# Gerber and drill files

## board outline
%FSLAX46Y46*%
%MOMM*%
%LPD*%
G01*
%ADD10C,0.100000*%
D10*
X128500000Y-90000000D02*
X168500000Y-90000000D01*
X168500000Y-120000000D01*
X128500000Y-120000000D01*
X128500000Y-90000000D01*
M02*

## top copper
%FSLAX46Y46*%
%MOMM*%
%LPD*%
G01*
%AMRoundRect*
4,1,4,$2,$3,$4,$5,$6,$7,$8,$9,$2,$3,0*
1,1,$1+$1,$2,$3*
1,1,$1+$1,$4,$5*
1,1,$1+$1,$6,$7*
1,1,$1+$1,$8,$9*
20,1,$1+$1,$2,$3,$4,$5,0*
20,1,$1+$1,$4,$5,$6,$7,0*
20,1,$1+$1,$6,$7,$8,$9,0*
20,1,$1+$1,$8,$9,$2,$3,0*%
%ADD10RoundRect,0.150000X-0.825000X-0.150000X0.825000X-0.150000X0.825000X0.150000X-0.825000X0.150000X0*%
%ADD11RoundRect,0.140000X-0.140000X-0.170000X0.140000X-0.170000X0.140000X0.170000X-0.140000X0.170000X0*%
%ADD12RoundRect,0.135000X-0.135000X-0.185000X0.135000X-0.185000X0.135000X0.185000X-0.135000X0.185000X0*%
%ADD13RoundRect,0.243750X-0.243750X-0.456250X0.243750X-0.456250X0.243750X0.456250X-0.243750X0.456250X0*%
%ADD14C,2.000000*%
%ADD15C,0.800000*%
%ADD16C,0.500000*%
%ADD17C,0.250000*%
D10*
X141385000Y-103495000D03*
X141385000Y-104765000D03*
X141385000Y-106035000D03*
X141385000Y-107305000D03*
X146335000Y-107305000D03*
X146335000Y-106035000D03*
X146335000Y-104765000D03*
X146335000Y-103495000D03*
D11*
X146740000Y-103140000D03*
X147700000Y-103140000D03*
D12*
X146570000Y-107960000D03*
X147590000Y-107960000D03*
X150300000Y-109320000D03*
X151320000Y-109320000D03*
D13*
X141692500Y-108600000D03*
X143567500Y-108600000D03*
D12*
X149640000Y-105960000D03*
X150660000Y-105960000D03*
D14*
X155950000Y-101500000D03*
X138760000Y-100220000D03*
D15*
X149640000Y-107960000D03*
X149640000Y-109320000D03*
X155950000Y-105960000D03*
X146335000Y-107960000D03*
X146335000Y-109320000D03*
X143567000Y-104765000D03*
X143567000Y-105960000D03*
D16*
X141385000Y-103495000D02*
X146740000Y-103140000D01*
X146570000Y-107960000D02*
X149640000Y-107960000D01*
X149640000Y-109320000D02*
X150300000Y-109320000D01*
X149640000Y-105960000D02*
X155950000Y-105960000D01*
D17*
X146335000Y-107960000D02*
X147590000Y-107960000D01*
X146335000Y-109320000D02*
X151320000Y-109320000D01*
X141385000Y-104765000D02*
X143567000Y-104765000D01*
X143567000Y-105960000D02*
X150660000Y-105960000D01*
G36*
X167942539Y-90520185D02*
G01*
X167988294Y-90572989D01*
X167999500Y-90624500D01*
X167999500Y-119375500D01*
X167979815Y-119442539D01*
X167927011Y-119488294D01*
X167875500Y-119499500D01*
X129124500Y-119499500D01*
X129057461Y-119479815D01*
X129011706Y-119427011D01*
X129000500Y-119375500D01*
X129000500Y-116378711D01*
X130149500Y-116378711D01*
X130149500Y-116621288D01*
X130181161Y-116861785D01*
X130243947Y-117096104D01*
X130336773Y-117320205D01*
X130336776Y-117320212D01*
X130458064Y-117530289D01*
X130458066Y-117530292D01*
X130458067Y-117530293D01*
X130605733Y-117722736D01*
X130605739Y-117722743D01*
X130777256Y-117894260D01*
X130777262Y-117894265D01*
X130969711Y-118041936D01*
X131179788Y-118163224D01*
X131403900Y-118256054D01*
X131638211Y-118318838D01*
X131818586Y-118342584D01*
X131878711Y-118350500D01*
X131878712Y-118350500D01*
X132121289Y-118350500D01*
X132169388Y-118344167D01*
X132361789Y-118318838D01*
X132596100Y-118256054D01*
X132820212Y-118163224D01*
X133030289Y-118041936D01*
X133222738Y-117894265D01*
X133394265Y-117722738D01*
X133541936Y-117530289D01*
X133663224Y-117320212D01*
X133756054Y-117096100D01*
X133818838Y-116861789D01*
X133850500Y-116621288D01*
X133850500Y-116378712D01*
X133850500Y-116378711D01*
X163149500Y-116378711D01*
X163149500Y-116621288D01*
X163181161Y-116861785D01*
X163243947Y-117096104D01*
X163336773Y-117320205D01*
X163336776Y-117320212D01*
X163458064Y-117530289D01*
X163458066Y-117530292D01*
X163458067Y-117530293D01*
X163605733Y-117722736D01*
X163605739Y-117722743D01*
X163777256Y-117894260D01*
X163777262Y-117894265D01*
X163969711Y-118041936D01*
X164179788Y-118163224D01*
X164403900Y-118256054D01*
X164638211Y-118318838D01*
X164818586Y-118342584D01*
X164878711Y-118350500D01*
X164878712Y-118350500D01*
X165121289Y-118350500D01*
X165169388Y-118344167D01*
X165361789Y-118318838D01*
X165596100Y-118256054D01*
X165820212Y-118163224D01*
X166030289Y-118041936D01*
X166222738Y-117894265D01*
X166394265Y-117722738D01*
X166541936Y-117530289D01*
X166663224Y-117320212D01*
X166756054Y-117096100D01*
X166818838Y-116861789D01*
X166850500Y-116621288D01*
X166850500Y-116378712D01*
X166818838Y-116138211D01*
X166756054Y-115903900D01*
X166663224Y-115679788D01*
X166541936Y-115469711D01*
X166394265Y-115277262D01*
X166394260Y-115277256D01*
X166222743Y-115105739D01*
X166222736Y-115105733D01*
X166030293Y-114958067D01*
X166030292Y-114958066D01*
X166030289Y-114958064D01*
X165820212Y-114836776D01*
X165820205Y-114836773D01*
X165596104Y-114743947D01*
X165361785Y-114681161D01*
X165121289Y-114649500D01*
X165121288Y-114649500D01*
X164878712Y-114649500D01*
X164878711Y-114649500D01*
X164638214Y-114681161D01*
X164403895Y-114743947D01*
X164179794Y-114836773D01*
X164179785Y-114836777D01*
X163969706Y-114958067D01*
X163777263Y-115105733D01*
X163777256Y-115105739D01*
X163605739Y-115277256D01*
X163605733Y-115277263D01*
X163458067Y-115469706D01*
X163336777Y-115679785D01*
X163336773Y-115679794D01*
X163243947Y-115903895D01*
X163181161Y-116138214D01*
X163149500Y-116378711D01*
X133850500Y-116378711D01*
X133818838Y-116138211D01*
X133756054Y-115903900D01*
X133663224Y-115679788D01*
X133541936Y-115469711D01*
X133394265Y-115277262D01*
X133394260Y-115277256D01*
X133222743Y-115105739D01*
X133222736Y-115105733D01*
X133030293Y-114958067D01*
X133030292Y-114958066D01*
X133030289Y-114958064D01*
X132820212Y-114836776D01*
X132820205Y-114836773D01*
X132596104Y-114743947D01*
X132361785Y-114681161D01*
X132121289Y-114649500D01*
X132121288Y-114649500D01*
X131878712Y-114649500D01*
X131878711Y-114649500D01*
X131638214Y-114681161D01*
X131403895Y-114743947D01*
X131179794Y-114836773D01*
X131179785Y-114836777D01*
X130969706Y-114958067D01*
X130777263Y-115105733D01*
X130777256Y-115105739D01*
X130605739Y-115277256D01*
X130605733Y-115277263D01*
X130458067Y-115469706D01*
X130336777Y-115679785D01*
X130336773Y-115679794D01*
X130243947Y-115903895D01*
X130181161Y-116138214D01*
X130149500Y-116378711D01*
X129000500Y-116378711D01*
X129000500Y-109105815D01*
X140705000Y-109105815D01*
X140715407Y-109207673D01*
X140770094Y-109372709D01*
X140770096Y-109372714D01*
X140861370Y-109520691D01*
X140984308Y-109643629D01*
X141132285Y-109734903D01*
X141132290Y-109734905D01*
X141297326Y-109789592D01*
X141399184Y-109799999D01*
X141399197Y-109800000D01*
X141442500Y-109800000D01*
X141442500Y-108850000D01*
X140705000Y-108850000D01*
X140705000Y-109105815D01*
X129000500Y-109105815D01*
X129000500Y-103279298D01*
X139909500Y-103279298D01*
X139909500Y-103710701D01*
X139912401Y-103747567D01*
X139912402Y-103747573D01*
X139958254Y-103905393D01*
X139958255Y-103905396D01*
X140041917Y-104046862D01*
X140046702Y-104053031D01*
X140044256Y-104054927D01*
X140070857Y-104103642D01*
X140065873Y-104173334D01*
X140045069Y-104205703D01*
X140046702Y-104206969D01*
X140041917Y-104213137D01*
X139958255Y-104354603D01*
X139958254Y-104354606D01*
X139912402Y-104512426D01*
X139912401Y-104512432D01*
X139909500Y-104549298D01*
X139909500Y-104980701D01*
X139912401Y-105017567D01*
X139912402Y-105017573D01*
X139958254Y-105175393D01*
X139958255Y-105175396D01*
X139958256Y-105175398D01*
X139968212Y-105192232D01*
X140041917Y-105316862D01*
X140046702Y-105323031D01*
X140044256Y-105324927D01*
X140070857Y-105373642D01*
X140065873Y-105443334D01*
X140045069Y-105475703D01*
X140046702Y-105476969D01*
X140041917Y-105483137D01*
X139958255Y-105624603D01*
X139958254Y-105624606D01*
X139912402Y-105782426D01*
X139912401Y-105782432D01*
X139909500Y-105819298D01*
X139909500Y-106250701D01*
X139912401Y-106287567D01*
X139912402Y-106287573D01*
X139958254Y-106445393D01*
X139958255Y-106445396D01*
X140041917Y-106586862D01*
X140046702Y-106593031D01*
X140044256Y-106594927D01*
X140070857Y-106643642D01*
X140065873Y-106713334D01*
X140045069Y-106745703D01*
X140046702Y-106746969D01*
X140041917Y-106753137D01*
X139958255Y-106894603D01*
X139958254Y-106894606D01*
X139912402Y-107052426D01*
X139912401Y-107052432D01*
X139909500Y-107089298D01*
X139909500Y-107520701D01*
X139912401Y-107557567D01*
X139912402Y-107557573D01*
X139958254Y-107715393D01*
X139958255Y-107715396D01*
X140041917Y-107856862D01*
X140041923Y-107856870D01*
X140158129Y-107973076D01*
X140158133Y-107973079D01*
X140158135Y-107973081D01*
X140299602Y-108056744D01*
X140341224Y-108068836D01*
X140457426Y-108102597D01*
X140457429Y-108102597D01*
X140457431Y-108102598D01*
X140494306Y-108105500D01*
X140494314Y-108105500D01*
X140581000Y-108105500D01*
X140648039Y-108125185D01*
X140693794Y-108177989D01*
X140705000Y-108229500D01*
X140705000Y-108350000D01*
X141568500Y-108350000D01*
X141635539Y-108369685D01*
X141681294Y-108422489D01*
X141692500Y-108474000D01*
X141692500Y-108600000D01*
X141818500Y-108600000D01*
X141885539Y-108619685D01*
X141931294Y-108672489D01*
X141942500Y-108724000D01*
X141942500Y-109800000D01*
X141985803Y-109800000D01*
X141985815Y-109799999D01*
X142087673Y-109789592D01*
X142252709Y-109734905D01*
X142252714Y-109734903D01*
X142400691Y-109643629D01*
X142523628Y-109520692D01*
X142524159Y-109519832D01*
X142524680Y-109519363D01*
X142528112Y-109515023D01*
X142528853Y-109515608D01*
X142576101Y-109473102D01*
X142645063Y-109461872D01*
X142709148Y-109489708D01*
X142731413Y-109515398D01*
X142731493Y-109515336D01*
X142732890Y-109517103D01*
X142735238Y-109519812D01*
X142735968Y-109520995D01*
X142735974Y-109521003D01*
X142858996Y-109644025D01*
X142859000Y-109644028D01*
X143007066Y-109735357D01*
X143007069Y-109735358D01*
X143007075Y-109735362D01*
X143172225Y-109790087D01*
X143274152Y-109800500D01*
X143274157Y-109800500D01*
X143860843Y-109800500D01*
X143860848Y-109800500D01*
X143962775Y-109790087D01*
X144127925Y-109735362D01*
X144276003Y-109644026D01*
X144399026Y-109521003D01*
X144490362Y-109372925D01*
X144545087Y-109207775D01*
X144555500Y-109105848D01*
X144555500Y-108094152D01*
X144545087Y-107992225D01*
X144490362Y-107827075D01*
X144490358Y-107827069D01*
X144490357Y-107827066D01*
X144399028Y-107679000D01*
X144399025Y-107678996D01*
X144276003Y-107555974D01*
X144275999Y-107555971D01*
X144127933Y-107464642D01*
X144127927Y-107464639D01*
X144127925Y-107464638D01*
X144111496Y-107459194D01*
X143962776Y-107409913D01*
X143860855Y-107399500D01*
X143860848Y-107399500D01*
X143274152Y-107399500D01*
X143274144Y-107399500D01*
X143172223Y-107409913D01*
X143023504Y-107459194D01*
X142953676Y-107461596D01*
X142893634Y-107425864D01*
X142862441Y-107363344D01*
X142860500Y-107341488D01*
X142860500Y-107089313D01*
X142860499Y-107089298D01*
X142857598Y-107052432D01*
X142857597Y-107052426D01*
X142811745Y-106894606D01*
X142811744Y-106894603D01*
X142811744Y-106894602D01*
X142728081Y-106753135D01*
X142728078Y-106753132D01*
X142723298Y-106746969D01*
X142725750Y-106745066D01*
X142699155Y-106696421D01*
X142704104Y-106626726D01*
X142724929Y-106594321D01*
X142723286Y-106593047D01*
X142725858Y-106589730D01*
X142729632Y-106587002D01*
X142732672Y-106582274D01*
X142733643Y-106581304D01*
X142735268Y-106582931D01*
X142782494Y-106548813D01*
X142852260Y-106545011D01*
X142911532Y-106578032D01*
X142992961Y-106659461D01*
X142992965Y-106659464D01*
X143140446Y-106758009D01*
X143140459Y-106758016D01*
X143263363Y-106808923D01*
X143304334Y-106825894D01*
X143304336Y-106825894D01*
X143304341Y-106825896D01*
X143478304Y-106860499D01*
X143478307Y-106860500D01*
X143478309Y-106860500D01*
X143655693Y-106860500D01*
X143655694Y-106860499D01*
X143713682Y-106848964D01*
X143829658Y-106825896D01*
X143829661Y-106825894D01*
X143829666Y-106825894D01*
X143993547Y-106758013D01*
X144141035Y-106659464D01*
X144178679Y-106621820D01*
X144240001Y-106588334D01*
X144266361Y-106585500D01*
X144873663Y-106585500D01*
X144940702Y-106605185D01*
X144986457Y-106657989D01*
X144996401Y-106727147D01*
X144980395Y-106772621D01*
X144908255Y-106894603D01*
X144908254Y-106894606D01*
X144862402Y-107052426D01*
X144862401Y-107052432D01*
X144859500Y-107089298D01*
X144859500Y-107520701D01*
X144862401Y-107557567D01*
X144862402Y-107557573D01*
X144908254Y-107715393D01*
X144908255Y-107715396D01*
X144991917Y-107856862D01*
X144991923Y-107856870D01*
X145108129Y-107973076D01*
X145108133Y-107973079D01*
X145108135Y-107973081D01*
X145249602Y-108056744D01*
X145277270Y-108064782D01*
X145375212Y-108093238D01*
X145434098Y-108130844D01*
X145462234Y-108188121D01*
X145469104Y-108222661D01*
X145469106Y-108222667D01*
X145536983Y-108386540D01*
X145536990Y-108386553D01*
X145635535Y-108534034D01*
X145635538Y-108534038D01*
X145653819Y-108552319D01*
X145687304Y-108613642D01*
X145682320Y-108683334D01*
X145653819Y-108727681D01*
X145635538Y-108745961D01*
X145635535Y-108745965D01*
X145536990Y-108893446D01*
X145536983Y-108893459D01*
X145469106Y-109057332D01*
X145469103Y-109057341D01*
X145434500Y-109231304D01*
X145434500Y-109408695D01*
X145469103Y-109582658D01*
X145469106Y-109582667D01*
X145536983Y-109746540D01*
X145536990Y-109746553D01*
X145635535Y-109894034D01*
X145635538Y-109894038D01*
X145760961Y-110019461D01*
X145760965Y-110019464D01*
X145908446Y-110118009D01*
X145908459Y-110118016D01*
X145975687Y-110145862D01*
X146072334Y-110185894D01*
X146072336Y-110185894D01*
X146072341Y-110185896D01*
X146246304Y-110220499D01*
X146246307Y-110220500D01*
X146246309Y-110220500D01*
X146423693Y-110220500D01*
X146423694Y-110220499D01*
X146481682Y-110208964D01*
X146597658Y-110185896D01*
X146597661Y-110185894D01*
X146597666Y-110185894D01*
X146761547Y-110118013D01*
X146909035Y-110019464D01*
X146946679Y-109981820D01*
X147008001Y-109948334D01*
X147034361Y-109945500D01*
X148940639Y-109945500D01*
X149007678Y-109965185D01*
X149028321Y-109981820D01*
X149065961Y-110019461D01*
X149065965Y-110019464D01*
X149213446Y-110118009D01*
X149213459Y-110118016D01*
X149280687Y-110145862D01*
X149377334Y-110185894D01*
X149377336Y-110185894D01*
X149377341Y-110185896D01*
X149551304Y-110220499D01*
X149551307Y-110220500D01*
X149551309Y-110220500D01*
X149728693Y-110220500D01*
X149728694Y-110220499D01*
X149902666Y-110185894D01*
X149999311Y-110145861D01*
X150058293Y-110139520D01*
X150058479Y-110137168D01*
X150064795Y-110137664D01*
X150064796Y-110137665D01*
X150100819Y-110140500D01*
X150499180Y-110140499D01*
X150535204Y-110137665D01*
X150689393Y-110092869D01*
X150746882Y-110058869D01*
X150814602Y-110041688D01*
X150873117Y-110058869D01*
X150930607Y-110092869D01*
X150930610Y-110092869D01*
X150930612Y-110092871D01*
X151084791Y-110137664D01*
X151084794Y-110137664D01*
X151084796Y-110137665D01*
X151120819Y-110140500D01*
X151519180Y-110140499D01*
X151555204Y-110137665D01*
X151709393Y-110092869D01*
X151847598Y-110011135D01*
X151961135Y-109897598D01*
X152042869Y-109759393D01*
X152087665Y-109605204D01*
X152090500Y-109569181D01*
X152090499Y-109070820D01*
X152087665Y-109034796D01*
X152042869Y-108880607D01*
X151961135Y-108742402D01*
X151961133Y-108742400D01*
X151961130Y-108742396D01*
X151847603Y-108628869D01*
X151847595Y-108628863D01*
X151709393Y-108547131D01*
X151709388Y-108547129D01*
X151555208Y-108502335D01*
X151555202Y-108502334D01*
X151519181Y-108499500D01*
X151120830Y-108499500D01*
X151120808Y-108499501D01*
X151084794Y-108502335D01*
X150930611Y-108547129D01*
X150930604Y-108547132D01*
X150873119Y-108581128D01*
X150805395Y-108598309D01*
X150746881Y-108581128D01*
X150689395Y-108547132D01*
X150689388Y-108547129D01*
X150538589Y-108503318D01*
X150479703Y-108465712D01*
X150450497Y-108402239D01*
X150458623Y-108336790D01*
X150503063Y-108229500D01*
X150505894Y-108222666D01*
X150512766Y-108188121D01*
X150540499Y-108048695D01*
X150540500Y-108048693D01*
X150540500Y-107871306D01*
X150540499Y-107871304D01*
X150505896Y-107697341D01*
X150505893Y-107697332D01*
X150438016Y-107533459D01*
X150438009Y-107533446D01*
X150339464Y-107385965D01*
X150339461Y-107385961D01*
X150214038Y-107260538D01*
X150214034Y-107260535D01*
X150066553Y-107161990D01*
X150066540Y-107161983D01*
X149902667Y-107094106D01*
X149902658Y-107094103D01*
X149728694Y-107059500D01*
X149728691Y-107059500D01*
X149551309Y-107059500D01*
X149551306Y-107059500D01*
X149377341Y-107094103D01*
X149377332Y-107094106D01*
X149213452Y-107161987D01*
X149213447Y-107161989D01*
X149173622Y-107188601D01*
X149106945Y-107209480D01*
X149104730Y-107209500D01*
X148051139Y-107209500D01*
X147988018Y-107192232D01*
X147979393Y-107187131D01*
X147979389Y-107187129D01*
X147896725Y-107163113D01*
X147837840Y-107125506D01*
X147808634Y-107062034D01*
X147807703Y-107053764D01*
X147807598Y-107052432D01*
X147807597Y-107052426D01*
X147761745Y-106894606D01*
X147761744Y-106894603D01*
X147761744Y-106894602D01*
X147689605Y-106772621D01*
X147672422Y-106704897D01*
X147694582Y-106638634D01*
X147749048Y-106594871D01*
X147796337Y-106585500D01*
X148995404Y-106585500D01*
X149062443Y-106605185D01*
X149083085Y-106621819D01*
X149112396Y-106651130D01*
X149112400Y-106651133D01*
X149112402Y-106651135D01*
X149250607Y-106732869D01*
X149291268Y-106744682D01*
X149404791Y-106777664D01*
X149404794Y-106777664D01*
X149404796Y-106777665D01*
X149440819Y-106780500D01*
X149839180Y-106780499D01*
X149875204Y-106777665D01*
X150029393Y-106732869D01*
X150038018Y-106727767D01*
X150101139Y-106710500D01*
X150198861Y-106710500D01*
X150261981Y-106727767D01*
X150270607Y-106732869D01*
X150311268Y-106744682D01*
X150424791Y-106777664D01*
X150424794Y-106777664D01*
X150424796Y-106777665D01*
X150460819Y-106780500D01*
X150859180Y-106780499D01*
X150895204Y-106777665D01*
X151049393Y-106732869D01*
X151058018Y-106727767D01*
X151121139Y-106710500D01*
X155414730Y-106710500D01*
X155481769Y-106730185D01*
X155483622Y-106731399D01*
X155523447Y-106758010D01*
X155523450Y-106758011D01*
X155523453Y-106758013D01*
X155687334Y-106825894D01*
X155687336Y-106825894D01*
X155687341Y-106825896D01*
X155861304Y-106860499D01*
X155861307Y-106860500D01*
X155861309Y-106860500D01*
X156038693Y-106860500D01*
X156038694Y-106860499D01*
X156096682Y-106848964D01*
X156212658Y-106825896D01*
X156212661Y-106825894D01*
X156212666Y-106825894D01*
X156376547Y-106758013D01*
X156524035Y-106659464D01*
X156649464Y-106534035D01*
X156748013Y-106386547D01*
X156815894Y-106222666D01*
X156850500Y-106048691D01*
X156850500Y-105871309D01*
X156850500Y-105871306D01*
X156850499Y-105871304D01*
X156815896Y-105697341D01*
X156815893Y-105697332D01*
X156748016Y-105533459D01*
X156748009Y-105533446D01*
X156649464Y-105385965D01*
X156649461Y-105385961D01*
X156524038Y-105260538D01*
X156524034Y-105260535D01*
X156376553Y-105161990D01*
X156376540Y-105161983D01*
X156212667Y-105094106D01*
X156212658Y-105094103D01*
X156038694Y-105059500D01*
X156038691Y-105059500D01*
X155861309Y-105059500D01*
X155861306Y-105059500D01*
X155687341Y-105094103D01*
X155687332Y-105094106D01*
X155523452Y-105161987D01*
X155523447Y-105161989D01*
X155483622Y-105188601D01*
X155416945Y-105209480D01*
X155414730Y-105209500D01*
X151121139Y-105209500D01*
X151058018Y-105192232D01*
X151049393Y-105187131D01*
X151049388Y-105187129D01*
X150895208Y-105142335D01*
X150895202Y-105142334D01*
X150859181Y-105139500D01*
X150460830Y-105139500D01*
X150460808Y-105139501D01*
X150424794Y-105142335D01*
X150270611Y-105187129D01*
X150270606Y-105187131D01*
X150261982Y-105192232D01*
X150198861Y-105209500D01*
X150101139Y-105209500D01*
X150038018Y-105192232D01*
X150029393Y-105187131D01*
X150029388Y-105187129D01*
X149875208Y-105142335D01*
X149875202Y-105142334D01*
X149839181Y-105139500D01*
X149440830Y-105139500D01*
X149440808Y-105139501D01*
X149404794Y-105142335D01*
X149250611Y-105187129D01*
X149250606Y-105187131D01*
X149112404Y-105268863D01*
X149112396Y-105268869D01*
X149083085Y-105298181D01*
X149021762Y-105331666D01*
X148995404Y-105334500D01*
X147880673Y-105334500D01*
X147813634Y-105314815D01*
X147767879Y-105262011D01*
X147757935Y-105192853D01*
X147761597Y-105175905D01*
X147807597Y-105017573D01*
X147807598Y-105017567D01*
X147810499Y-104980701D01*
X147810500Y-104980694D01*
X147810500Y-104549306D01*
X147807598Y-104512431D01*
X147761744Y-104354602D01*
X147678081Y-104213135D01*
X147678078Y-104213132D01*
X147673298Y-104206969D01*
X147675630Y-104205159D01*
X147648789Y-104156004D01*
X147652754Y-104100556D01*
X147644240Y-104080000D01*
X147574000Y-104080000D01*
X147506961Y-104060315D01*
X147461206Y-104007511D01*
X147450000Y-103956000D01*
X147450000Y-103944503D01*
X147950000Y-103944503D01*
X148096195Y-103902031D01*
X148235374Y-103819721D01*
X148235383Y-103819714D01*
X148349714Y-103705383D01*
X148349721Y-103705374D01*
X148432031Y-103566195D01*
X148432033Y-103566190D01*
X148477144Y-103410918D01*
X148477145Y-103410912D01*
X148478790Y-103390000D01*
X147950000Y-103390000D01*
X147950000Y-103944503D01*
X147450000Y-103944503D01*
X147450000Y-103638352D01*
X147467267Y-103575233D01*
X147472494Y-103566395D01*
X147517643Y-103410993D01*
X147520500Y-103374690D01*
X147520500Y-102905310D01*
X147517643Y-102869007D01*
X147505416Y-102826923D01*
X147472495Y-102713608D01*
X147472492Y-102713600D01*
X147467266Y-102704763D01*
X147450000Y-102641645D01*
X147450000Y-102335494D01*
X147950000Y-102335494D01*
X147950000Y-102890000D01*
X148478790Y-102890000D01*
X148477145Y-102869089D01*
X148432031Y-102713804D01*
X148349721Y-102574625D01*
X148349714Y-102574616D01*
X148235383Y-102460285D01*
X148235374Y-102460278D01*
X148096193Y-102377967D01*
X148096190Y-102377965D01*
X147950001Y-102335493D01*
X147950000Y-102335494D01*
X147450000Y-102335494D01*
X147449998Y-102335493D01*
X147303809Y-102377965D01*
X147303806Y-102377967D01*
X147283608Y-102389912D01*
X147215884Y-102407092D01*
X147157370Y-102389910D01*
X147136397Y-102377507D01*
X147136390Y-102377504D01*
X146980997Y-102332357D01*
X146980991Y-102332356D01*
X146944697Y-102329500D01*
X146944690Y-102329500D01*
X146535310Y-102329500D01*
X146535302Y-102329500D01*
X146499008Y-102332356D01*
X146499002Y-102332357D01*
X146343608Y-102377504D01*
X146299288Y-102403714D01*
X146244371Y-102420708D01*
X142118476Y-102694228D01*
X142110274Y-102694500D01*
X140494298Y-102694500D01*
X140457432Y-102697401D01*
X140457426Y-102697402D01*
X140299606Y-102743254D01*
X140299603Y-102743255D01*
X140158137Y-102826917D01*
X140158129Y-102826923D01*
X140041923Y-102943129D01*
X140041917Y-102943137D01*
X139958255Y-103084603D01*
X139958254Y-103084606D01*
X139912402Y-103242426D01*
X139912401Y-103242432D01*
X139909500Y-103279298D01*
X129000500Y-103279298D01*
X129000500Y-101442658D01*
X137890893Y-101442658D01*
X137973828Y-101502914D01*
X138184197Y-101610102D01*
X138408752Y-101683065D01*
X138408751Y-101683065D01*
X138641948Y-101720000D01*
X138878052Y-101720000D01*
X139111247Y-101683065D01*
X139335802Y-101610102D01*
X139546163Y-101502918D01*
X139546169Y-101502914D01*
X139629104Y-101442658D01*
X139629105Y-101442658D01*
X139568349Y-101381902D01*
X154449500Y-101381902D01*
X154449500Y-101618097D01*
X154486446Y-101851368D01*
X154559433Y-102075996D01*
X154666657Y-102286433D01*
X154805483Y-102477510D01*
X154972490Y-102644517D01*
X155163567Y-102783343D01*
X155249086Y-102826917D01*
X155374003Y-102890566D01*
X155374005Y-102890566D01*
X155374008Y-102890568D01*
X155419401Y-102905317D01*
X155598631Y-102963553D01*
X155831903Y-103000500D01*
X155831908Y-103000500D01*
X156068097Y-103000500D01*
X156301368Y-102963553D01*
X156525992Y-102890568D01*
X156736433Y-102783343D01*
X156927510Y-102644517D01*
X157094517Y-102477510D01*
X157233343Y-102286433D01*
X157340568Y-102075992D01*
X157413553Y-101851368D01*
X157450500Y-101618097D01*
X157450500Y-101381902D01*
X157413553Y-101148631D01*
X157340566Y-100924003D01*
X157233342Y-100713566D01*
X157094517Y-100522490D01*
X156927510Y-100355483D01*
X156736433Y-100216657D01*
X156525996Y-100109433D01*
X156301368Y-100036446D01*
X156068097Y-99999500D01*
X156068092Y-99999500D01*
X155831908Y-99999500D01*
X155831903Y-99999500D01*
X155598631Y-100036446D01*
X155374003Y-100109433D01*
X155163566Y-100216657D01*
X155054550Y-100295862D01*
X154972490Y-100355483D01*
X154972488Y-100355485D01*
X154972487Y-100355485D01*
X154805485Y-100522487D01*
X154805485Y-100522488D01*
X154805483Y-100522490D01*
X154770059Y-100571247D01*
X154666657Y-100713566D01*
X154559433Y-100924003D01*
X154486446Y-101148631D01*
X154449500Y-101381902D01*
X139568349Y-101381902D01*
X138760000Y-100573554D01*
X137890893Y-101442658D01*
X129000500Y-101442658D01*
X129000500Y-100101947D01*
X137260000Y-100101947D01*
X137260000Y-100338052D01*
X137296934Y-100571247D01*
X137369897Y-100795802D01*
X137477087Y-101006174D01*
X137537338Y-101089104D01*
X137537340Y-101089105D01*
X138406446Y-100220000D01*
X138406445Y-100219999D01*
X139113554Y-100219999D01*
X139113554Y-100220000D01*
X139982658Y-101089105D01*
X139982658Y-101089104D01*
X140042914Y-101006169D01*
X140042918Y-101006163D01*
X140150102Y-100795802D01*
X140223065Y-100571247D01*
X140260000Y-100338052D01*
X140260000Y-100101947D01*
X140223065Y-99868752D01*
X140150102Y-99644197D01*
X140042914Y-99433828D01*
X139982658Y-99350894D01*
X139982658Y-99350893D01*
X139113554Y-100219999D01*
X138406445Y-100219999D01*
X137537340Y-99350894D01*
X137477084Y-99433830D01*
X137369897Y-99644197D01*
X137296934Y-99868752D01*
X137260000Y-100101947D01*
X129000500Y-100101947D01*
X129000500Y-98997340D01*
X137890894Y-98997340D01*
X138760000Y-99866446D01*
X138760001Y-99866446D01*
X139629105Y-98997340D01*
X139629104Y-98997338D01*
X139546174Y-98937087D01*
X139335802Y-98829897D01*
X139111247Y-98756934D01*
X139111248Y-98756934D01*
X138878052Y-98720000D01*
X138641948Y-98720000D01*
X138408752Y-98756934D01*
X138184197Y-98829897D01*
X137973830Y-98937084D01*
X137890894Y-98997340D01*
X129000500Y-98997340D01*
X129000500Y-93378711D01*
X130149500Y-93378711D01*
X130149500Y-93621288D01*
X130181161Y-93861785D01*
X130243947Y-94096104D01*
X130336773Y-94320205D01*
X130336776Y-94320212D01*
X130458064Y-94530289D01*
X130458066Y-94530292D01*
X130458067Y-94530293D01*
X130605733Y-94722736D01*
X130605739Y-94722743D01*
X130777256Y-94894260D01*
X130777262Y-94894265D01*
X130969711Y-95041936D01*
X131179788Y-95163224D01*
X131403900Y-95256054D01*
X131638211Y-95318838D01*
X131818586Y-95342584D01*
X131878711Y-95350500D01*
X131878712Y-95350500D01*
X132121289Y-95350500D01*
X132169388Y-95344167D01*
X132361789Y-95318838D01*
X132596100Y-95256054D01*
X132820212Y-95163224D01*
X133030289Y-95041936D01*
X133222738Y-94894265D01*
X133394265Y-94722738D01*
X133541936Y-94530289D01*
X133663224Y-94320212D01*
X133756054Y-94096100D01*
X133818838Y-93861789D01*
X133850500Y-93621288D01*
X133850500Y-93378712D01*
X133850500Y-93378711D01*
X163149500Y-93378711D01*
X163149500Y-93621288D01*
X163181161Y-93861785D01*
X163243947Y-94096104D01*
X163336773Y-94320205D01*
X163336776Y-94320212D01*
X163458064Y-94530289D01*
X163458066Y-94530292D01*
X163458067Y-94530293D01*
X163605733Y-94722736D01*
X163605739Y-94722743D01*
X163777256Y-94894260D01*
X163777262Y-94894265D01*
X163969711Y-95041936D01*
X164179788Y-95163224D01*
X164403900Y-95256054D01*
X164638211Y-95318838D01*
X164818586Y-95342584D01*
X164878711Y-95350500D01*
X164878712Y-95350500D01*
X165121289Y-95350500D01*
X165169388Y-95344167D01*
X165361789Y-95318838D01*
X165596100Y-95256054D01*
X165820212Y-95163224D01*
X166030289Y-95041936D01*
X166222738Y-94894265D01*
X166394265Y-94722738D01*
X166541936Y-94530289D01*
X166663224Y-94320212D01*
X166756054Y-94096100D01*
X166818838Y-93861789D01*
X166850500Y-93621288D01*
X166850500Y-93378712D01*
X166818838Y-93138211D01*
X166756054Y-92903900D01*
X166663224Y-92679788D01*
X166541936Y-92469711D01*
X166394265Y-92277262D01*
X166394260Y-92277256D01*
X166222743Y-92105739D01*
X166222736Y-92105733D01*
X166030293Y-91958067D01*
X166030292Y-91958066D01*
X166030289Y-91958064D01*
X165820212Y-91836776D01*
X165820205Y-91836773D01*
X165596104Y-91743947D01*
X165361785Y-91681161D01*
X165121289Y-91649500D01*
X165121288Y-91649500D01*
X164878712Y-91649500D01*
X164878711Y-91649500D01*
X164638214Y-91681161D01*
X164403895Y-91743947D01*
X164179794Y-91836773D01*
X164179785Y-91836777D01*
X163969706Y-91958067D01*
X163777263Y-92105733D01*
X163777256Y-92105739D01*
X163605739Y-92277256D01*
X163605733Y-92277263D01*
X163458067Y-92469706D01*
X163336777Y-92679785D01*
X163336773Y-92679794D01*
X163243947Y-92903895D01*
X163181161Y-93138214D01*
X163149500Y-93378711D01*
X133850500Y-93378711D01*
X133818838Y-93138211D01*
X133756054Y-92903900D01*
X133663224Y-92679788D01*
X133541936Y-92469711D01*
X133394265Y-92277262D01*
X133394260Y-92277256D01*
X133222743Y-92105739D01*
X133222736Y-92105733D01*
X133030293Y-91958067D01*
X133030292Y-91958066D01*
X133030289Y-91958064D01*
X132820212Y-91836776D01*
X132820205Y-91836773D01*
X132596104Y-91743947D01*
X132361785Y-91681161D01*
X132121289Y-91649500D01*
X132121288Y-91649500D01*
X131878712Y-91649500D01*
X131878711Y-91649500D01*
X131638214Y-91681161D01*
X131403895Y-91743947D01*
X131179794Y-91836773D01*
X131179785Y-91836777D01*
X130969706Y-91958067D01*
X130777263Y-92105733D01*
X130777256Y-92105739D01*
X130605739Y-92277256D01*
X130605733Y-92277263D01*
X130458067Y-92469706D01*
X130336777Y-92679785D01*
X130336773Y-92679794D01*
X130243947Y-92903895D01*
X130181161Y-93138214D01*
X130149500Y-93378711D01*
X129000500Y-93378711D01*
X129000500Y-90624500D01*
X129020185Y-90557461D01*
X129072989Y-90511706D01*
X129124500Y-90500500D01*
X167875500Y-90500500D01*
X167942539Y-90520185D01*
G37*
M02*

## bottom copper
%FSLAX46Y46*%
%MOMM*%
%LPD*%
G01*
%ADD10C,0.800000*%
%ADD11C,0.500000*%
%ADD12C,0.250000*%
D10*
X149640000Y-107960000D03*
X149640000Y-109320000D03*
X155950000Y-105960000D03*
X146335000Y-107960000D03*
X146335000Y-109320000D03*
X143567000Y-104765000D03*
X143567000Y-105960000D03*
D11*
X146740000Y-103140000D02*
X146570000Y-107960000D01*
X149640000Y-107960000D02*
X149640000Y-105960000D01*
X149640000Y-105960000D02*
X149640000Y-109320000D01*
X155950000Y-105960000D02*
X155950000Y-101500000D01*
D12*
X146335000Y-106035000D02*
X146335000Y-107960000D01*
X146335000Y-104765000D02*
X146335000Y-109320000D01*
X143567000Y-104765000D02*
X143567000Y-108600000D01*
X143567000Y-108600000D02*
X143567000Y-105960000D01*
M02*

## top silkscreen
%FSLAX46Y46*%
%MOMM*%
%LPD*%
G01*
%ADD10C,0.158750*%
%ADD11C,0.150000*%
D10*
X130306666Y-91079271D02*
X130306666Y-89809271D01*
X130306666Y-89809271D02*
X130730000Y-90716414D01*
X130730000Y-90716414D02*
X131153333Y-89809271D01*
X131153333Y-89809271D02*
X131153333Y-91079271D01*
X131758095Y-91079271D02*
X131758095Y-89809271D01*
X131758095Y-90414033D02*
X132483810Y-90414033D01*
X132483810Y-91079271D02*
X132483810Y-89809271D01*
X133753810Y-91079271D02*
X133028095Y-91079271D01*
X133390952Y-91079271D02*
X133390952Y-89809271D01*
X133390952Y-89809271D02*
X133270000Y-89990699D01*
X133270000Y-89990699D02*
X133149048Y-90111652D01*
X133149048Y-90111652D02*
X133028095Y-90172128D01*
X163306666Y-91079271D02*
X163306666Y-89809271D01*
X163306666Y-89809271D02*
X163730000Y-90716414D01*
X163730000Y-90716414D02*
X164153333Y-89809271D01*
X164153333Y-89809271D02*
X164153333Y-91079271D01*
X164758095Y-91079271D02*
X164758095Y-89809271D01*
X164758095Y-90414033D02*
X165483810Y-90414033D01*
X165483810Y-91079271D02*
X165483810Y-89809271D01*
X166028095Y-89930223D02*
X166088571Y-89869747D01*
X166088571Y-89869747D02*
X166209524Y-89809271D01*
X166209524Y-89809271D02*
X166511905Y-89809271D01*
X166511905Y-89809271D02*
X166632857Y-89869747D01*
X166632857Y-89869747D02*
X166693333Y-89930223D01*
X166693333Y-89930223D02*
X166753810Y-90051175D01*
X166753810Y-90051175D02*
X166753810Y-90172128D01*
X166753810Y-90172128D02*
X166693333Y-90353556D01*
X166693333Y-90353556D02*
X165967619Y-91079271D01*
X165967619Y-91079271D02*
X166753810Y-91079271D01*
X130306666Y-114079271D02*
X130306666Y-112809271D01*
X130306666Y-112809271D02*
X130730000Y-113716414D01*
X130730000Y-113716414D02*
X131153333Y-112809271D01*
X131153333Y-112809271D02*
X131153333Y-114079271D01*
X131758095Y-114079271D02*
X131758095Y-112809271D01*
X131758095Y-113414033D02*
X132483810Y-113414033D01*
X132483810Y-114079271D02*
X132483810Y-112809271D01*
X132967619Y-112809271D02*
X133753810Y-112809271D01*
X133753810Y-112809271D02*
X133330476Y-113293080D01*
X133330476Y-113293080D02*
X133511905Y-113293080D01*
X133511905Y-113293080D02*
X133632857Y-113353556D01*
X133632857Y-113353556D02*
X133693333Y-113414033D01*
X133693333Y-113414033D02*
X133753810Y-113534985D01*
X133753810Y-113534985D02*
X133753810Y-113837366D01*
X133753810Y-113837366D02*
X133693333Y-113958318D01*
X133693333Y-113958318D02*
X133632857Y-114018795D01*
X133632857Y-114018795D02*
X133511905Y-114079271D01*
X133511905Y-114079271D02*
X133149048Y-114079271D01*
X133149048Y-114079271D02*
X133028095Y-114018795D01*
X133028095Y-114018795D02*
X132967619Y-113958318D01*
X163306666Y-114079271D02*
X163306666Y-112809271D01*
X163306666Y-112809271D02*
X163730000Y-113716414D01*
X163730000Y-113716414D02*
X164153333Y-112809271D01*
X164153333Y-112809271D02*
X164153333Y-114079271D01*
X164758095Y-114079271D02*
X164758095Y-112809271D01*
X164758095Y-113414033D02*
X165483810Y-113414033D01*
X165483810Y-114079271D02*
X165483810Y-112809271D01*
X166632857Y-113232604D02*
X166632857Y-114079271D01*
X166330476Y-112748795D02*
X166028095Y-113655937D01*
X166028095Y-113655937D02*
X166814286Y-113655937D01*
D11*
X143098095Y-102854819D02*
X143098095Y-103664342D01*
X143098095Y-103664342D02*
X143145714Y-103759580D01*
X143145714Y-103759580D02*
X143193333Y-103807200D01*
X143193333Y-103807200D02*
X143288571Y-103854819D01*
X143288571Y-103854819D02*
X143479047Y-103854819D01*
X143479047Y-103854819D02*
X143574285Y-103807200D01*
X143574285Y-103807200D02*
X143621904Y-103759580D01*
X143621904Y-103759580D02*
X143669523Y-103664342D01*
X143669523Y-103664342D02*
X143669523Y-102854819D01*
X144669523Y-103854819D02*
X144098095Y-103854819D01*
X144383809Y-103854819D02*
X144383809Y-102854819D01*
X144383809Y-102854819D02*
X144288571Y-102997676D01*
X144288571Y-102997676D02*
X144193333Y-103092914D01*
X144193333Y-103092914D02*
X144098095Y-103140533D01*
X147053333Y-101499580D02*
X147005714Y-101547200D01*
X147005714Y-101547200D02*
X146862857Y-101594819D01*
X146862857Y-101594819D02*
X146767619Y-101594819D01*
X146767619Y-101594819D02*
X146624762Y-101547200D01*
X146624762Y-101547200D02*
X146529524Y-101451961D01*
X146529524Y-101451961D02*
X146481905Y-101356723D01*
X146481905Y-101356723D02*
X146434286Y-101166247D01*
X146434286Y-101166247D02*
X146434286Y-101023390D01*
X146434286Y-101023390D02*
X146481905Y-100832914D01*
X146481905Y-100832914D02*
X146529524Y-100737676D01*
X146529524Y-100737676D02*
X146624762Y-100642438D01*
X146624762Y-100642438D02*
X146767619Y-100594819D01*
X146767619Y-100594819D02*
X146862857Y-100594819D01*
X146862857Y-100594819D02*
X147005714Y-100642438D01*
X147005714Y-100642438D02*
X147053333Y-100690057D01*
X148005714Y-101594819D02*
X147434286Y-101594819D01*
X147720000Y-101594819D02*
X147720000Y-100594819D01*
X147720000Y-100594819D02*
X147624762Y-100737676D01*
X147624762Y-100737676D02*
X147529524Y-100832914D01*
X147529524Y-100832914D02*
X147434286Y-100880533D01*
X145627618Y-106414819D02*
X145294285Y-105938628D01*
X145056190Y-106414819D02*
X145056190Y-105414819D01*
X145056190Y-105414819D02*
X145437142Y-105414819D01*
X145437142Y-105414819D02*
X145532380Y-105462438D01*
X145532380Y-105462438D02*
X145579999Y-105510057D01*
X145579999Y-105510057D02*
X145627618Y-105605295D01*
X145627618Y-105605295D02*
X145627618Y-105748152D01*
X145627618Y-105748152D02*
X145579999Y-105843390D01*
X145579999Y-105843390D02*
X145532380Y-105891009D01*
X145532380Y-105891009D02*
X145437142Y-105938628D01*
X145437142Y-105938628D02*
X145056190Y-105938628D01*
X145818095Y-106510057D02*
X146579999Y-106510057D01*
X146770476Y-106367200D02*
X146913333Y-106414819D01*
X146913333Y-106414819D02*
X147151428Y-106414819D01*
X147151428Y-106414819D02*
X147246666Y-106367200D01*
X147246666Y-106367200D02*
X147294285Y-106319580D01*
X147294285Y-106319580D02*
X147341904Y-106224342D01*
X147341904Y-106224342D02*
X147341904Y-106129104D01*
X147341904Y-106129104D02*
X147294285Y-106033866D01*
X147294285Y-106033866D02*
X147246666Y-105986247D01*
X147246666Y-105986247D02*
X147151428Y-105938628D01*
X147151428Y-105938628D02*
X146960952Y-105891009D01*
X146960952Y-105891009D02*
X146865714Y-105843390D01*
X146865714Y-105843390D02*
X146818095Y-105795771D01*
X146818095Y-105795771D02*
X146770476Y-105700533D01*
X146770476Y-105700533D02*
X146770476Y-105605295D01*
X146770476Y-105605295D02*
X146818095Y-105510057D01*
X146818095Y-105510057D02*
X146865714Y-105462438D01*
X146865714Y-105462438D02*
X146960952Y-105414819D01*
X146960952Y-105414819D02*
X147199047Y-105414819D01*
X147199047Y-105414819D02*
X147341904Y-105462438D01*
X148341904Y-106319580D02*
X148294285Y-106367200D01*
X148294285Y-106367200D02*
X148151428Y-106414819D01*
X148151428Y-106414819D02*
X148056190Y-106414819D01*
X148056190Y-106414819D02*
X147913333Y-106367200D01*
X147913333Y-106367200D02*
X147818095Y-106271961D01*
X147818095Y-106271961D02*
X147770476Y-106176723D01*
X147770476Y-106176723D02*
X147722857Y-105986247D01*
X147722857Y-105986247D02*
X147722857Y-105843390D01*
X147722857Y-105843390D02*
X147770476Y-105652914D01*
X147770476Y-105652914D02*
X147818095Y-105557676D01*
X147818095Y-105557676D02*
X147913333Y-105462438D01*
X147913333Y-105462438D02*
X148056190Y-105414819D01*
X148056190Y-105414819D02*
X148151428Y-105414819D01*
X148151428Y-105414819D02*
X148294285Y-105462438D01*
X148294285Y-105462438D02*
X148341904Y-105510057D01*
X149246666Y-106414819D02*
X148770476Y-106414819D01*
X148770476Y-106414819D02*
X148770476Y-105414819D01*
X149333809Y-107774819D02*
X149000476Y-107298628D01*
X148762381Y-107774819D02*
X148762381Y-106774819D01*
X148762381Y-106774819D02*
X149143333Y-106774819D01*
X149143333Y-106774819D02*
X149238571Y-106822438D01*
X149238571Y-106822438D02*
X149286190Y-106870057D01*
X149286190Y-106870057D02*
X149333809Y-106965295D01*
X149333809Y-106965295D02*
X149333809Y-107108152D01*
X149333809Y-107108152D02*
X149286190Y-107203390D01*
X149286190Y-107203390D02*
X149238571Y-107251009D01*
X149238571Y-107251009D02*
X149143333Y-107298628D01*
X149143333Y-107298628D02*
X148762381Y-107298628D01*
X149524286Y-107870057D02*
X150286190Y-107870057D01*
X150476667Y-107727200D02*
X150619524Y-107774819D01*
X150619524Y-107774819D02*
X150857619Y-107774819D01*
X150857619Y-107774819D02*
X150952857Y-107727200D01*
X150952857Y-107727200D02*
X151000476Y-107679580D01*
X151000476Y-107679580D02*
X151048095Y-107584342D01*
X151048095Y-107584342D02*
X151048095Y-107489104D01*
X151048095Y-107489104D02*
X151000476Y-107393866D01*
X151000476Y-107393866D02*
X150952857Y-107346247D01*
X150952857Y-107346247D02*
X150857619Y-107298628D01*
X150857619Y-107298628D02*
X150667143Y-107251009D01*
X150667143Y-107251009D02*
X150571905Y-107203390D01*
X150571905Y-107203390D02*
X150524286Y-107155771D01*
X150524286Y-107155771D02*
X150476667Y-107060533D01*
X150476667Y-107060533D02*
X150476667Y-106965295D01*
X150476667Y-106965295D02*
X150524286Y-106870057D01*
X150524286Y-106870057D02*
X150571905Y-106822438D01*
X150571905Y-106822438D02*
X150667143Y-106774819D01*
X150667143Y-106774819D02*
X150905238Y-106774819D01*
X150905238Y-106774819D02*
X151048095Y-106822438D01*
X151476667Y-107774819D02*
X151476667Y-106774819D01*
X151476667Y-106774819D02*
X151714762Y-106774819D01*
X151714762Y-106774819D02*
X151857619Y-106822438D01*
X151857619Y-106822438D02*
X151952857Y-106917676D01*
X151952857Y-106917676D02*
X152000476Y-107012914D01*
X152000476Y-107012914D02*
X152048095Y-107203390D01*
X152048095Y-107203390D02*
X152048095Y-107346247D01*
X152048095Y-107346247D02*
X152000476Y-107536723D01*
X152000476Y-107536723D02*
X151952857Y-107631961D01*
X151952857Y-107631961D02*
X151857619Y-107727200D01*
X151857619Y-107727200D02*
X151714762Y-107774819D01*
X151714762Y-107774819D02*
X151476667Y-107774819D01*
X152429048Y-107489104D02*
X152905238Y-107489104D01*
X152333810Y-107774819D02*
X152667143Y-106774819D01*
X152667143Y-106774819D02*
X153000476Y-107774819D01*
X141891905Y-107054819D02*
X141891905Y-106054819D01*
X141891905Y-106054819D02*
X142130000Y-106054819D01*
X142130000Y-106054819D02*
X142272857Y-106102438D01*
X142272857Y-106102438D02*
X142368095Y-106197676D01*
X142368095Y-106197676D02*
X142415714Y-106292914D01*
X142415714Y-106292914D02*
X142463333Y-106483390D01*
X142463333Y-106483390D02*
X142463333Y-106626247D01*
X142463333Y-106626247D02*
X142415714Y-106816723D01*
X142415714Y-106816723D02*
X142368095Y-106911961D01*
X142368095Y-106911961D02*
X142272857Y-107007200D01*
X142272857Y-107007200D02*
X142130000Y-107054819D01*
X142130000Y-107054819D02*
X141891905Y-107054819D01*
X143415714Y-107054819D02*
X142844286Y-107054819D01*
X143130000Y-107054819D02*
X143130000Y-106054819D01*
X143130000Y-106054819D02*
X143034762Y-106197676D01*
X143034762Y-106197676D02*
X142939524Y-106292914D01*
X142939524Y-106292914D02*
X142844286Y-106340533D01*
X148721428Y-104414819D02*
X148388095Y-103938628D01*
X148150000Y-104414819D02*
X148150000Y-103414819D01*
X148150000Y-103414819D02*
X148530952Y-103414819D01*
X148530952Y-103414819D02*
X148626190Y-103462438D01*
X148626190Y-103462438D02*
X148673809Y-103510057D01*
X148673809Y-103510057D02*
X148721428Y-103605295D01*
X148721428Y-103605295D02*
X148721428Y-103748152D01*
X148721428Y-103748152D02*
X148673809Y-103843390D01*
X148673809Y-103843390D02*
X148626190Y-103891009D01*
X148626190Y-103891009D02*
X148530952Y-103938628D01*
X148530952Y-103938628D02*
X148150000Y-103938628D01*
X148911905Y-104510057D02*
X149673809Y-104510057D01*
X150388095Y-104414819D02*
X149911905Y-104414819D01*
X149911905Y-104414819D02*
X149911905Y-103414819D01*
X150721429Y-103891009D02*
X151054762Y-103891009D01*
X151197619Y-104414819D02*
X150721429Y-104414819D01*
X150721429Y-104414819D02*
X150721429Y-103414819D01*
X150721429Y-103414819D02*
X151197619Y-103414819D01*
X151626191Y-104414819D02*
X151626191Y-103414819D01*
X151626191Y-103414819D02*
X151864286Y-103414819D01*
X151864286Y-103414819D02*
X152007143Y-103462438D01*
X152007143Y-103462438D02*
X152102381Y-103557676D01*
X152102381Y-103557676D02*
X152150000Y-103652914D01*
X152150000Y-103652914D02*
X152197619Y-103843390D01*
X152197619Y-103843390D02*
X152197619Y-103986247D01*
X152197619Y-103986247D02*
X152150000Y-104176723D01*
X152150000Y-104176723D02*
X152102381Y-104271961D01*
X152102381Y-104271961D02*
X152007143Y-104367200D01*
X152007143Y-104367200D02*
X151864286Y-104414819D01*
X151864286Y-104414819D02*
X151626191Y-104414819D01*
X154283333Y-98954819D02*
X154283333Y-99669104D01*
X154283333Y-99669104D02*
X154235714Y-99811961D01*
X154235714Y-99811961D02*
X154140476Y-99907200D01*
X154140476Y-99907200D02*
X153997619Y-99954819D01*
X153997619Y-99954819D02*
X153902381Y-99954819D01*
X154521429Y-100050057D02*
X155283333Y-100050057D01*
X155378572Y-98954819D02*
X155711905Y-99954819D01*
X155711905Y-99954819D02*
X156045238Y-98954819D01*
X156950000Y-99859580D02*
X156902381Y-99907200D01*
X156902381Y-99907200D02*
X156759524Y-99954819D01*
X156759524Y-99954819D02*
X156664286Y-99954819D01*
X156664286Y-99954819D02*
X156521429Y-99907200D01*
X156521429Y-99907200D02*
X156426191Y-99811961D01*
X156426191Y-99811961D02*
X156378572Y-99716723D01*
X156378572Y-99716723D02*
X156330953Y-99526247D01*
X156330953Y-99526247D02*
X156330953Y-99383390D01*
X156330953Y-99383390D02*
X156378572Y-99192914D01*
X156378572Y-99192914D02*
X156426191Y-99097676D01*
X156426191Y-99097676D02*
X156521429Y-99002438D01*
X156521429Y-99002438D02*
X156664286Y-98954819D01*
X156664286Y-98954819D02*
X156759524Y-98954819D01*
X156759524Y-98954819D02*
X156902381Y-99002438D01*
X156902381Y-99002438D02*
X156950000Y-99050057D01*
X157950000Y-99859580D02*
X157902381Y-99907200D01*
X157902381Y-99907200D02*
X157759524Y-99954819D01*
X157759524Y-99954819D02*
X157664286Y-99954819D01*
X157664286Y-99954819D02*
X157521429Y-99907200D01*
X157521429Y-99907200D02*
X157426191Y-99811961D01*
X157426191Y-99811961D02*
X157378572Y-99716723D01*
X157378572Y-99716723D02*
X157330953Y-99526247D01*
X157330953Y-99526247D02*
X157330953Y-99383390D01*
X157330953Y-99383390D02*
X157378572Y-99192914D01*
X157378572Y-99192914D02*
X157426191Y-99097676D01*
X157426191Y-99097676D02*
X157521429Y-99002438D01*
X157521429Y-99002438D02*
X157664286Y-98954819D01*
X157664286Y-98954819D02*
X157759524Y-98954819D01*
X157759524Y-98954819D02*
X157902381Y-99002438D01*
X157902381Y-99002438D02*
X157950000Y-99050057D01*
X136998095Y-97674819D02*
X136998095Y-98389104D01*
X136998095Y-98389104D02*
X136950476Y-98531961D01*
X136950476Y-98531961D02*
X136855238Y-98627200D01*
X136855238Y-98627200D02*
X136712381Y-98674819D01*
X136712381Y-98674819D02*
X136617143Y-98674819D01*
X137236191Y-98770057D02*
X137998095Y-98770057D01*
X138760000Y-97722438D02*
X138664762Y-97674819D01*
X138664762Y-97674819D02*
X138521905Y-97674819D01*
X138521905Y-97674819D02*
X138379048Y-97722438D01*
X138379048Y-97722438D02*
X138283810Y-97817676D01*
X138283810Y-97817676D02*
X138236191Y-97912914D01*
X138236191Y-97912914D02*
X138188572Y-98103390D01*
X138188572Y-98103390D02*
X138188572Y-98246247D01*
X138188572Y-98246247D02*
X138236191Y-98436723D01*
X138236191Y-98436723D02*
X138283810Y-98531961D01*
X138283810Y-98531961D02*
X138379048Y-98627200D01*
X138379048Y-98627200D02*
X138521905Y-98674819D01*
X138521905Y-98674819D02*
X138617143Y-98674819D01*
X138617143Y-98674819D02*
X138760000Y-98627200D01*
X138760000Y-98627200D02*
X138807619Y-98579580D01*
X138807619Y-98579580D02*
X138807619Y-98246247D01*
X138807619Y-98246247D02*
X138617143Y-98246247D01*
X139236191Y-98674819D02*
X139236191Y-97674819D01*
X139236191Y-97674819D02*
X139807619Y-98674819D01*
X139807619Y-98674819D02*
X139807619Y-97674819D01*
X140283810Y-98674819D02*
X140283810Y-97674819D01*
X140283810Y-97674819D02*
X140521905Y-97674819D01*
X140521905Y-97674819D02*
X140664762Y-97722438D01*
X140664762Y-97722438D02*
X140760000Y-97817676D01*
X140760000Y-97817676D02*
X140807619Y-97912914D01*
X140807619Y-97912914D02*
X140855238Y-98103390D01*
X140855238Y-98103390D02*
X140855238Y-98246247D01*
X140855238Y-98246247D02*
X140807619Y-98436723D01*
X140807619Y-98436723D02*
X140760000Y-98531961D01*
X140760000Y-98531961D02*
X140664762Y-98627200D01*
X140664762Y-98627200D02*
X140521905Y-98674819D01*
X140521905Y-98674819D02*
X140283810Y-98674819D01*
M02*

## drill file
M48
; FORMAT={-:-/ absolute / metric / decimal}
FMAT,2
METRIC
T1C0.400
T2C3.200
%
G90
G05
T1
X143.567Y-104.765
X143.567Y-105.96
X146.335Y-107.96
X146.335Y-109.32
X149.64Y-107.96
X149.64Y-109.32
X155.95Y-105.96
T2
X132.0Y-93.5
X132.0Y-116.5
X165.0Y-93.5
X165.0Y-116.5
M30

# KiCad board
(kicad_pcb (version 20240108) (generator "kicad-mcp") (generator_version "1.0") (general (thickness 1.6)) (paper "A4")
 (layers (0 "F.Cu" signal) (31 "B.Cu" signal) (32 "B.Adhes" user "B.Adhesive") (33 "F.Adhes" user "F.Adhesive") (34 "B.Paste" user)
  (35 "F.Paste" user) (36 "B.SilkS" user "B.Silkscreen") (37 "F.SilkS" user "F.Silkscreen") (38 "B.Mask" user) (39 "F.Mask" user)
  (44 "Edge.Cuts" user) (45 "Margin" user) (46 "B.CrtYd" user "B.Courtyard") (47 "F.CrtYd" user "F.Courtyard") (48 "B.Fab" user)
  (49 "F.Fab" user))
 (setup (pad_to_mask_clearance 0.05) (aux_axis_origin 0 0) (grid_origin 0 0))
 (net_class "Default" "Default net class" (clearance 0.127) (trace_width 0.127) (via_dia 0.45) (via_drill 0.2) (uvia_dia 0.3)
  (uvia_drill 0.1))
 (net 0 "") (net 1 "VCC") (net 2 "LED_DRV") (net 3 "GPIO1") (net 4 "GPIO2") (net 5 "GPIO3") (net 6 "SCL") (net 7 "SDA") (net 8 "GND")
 (gr_rect (start 128.5 90.0) (end 168.5 120.0) (layer "Edge.Cuts") (stroke (width 0.1) (type default)))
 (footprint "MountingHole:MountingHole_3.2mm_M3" (layer "F.Cu") (at 132.0 93.5)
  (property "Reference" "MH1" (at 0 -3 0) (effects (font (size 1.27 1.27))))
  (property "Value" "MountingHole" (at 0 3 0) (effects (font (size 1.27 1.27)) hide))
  (pad "" np_thru_hole circle (at 0 0) (size 3.2 3.2) (drill 3.2) (layers "*.Cu" "*.Mask")))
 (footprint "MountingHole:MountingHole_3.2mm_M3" (layer "F.Cu") (at 165.0 93.5)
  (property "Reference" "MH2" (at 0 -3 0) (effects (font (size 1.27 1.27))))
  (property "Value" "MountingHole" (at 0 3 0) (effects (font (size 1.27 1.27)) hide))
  (pad "" np_thru_hole circle (at 0 0) (size 3.2 3.2) (drill 3.2) (layers "*.Cu" "*.Mask")))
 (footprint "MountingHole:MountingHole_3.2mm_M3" (layer "F.Cu") (at 132.0 116.5)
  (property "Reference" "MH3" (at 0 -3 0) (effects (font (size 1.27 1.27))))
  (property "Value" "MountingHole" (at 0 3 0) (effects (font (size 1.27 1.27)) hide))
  (pad "" np_thru_hole circle (at 0 0) (size 3.2 3.2) (drill 3.2) (layers "*.Cu" "*.Mask")))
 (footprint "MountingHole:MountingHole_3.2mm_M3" (layer "F.Cu") (at 165.0 116.5)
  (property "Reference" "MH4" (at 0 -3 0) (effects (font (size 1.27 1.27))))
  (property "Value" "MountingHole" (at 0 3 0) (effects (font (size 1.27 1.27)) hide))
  (pad "" np_thru_hole circle (at 0 0) (size 3.2 3.2) (drill 3.2) (layers "*.Cu" "*.Mask")))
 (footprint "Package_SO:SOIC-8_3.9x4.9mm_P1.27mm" (layer "F.Cu") (at 143.86 105.4)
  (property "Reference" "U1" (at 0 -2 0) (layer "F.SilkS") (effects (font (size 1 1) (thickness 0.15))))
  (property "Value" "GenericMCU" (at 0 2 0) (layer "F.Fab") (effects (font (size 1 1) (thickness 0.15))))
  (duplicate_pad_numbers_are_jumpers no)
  (pad "1" smd roundrect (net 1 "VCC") (at -2.475 -1.905) (size 1.95 0.6) (layers "F.Cu" "F.Mask" "F.Paste") (roundrect_rratio 0.25))
  (pad "2" smd roundrect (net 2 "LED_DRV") (at -2.475 -0.635) (size 1.95 0.6) (layers "F.Cu" "F.Mask" "F.Paste") (roundrect_rratio 0.25))
  (pad "3" smd roundrect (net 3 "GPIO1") (at -2.475 0.635) (size 1.95 0.6) (layers "F.Cu" "F.Mask" "F.Paste") (roundrect_rratio 0.25))
  (pad "4" smd roundrect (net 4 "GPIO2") (at -2.475 1.905) (size 1.95 0.6) (layers "F.Cu" "F.Mask" "F.Paste") (roundrect_rratio 0.25))
  (pad "5" smd roundrect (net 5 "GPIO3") (at 2.475 1.905) (size 1.95 0.6) (layers "F.Cu" "F.Mask" "F.Paste") (roundrect_rratio 0.25))
  (pad "6" smd roundrect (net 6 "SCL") (at 2.475 0.635) (size 1.95 0.6) (layers "F.Cu" "F.Mask" "F.Paste") (roundrect_rratio 0.25))
  (pad "7" smd roundrect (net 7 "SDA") (at 2.475 -0.635) (size 1.95 0.6) (layers "F.Cu" "F.Mask" "F.Paste") (roundrect_rratio 0.25))
  (pad "8" smd roundrect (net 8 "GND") (at 2.475 -1.905) (size 1.95 0.6) (layers "F.Cu" "F.Mask" "F.Paste") (roundrect_rratio 0.25)))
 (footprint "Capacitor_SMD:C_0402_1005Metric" (layer "F.Cu") (at 147.22 103.14)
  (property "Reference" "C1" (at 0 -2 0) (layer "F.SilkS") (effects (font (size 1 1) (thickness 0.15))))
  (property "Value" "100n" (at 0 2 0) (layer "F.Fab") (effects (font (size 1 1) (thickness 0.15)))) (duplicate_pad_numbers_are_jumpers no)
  (pad "1" smd roundrect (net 1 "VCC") (at -0.48 0) (size 0.56 0.62) (layers "F.Cu" "F.Mask" "F.Paste") (roundrect_rratio 0.25))
  (pad "2" smd roundrect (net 8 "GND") (at 0.48 0) (size 0.56 0.62) (layers "F.Cu" "F.Mask" "F.Paste") (roundrect_rratio 0.25)))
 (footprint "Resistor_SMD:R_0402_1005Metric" (layer "F.Cu") (at 147.07999999999998 107.96000000000001)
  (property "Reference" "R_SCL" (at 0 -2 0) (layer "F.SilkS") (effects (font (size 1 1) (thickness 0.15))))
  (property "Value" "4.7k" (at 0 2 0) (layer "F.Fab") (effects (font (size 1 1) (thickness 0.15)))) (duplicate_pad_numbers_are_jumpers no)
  (pad "1" smd roundrect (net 1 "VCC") (at -0.51 0) (size 0.54 0.64) (layers "F.Cu" "F.Mask" "F.Paste") (roundrect_rratio 0.25))
  (pad "2" smd roundrect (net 6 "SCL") (at 0.51 0) (size 0.54 0.64) (layers "F.Cu" "F.Mask" "F.Paste") (roundrect_rratio 0.25)))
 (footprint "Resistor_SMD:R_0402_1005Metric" (layer "F.Cu") (at 150.81 109.32)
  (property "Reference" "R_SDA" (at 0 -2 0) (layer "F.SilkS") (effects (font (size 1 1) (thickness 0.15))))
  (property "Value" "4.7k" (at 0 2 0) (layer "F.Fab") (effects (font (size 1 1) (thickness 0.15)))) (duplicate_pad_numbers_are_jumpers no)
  (pad "1" smd roundrect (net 1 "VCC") (at -0.51 0) (size 0.54 0.64) (layers "F.Cu" "F.Mask" "F.Paste") (roundrect_rratio 0.25))
  (pad "2" smd roundrect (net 7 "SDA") (at 0.51 0) (size 0.54 0.64) (layers "F.Cu" "F.Mask" "F.Paste") (roundrect_rratio 0.25)))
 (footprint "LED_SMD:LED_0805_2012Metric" (layer "F.Cu") (at 142.63 108.6)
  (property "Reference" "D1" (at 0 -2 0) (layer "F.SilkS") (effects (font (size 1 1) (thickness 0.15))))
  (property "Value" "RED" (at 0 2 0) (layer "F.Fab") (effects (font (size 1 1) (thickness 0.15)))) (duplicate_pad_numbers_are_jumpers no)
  (pad "1" smd roundrect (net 8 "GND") (at -0.9375 0) (size 0.975 1.4) (layers "F.Cu" "F.Mask" "F.Paste") (roundrect_rratio 0.25))
  (pad "2" smd roundrect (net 2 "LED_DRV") (at 0.9375 0) (size 0.975 1.4) (layers "F.Cu" "F.Mask" "F.Paste") (roundrect_rratio 0.25)))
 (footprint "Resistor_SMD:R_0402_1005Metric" (layer "F.Cu") (at 150.15 105.96000000000001)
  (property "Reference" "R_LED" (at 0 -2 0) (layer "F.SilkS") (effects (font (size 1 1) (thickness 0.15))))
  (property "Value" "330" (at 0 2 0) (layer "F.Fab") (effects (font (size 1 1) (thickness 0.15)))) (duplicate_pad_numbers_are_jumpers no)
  (pad "1" smd roundrect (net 1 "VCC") (at -0.51 0) (size 0.54 0.64) (layers "F.Cu" "F.Mask" "F.Paste") (roundrect_rratio 0.25))
  (pad "2" smd roundrect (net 2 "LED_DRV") (at 0.51 0) (size 0.54 0.64) (layers "F.Cu" "F.Mask" "F.Paste") (roundrect_rratio 0.25)))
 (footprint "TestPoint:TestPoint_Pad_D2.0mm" (layer "F.Cu") (at 155.95 101.5) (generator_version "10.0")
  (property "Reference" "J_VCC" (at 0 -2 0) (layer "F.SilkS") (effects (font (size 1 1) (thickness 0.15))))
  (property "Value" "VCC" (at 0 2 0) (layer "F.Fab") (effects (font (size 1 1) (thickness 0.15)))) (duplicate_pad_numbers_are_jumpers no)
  (pad "1" smd circle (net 1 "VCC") (at 0 0) (size 2 2) (layers "F.Cu" "F.Mask")))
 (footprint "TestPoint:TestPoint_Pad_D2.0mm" (layer "F.Cu") (at 138.76 100.22) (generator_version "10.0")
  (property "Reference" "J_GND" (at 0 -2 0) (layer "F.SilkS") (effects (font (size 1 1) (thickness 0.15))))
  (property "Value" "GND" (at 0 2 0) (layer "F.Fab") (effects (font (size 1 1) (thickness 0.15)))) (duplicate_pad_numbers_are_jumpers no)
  (pad "1" smd circle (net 8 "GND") (at 0 0) (size 2 2) (layers "F.Cu" "F.Mask")))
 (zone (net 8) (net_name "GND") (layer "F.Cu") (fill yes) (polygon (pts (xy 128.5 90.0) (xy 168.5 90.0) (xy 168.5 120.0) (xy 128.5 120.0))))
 (segment (start 141.385 103.495) (end 146.740 103.140) (width 0.5) (layer "F.Cu") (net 1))
 (segment (start 146.740 103.140) (end 146.570 107.960) (width 0.5) (layer "B.Cu") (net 1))
 (segment (start 146.570 107.960) (end 149.640 107.960) (width 0.5) (layer "F.Cu") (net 1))
 (via (at 149.640 107.960) (size 0.8) (drill 0.4) (layers "F.Cu" "B.Cu") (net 1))
 (segment (start 149.640 107.960) (end 149.640 105.960) (width 0.5) (layer "B.Cu") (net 1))
 (segment (start 149.640 105.960) (end 149.640 109.320) (width 0.5) (layer "B.Cu") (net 1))
 (via (at 149.640 109.320) (size 0.8) (drill 0.4) (layers "F.Cu" "B.Cu") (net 1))
 (segment (start 149.640 109.320) (end 150.300 109.320) (width 0.5) (layer "F.Cu") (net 1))
 (segment (start 149.640 105.960) (end 155.950 105.960) (width 0.5) (layer "F.Cu") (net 1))
 (via (at 155.950 105.960) (size 0.8) (drill 0.4) (layers "F.Cu" "B.Cu") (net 1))
 (segment (start 155.950 105.960) (end 155.950 101.500) (width 0.5) (layer "B.Cu") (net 1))
 (segment (start 146.335 106.035) (end 146.335 107.960) (width 0.25) (layer "B.Cu") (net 6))
 (via (at 146.335 107.960) (size 0.8) (drill 0.4) (layers "F.Cu" "B.Cu") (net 6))
 (segment (start 146.335 107.960) (end 147.590 107.960) (width 0.25) (layer "F.Cu") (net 6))
 (segment (start 146.335 104.765) (end 146.335 109.320) (width 0.25) (layer "B.Cu") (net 7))
 (via (at 146.335 109.320) (size 0.8) (drill 0.4) (layers "F.Cu" "B.Cu") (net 7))
 (segment (start 146.335 109.320) (end 151.320 109.320) (width 0.25) (layer "F.Cu") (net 7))
 (segment (start 141.385 104.765) (end 143.567 104.765) (width 0.25) (layer "F.Cu") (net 2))
 (via (at 143.567 104.765) (size 0.8) (drill 0.4) (layers "F.Cu" "B.Cu") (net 2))
 (segment (start 143.567 104.765) (end 143.567 108.600) (width 0.25) (layer "B.Cu") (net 2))
 (segment (start 143.567 108.600) (end 143.567 105.960) (width 0.25) (layer "B.Cu") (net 2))
 (via (at 143.567 105.960) (size 0.8) (drill 0.4) (layers "F.Cu" "B.Cu") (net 2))
 (segment (start 143.567 105.960) (end 150.660 105.960) (width 0.25) (layer "F.Cu") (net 2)))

